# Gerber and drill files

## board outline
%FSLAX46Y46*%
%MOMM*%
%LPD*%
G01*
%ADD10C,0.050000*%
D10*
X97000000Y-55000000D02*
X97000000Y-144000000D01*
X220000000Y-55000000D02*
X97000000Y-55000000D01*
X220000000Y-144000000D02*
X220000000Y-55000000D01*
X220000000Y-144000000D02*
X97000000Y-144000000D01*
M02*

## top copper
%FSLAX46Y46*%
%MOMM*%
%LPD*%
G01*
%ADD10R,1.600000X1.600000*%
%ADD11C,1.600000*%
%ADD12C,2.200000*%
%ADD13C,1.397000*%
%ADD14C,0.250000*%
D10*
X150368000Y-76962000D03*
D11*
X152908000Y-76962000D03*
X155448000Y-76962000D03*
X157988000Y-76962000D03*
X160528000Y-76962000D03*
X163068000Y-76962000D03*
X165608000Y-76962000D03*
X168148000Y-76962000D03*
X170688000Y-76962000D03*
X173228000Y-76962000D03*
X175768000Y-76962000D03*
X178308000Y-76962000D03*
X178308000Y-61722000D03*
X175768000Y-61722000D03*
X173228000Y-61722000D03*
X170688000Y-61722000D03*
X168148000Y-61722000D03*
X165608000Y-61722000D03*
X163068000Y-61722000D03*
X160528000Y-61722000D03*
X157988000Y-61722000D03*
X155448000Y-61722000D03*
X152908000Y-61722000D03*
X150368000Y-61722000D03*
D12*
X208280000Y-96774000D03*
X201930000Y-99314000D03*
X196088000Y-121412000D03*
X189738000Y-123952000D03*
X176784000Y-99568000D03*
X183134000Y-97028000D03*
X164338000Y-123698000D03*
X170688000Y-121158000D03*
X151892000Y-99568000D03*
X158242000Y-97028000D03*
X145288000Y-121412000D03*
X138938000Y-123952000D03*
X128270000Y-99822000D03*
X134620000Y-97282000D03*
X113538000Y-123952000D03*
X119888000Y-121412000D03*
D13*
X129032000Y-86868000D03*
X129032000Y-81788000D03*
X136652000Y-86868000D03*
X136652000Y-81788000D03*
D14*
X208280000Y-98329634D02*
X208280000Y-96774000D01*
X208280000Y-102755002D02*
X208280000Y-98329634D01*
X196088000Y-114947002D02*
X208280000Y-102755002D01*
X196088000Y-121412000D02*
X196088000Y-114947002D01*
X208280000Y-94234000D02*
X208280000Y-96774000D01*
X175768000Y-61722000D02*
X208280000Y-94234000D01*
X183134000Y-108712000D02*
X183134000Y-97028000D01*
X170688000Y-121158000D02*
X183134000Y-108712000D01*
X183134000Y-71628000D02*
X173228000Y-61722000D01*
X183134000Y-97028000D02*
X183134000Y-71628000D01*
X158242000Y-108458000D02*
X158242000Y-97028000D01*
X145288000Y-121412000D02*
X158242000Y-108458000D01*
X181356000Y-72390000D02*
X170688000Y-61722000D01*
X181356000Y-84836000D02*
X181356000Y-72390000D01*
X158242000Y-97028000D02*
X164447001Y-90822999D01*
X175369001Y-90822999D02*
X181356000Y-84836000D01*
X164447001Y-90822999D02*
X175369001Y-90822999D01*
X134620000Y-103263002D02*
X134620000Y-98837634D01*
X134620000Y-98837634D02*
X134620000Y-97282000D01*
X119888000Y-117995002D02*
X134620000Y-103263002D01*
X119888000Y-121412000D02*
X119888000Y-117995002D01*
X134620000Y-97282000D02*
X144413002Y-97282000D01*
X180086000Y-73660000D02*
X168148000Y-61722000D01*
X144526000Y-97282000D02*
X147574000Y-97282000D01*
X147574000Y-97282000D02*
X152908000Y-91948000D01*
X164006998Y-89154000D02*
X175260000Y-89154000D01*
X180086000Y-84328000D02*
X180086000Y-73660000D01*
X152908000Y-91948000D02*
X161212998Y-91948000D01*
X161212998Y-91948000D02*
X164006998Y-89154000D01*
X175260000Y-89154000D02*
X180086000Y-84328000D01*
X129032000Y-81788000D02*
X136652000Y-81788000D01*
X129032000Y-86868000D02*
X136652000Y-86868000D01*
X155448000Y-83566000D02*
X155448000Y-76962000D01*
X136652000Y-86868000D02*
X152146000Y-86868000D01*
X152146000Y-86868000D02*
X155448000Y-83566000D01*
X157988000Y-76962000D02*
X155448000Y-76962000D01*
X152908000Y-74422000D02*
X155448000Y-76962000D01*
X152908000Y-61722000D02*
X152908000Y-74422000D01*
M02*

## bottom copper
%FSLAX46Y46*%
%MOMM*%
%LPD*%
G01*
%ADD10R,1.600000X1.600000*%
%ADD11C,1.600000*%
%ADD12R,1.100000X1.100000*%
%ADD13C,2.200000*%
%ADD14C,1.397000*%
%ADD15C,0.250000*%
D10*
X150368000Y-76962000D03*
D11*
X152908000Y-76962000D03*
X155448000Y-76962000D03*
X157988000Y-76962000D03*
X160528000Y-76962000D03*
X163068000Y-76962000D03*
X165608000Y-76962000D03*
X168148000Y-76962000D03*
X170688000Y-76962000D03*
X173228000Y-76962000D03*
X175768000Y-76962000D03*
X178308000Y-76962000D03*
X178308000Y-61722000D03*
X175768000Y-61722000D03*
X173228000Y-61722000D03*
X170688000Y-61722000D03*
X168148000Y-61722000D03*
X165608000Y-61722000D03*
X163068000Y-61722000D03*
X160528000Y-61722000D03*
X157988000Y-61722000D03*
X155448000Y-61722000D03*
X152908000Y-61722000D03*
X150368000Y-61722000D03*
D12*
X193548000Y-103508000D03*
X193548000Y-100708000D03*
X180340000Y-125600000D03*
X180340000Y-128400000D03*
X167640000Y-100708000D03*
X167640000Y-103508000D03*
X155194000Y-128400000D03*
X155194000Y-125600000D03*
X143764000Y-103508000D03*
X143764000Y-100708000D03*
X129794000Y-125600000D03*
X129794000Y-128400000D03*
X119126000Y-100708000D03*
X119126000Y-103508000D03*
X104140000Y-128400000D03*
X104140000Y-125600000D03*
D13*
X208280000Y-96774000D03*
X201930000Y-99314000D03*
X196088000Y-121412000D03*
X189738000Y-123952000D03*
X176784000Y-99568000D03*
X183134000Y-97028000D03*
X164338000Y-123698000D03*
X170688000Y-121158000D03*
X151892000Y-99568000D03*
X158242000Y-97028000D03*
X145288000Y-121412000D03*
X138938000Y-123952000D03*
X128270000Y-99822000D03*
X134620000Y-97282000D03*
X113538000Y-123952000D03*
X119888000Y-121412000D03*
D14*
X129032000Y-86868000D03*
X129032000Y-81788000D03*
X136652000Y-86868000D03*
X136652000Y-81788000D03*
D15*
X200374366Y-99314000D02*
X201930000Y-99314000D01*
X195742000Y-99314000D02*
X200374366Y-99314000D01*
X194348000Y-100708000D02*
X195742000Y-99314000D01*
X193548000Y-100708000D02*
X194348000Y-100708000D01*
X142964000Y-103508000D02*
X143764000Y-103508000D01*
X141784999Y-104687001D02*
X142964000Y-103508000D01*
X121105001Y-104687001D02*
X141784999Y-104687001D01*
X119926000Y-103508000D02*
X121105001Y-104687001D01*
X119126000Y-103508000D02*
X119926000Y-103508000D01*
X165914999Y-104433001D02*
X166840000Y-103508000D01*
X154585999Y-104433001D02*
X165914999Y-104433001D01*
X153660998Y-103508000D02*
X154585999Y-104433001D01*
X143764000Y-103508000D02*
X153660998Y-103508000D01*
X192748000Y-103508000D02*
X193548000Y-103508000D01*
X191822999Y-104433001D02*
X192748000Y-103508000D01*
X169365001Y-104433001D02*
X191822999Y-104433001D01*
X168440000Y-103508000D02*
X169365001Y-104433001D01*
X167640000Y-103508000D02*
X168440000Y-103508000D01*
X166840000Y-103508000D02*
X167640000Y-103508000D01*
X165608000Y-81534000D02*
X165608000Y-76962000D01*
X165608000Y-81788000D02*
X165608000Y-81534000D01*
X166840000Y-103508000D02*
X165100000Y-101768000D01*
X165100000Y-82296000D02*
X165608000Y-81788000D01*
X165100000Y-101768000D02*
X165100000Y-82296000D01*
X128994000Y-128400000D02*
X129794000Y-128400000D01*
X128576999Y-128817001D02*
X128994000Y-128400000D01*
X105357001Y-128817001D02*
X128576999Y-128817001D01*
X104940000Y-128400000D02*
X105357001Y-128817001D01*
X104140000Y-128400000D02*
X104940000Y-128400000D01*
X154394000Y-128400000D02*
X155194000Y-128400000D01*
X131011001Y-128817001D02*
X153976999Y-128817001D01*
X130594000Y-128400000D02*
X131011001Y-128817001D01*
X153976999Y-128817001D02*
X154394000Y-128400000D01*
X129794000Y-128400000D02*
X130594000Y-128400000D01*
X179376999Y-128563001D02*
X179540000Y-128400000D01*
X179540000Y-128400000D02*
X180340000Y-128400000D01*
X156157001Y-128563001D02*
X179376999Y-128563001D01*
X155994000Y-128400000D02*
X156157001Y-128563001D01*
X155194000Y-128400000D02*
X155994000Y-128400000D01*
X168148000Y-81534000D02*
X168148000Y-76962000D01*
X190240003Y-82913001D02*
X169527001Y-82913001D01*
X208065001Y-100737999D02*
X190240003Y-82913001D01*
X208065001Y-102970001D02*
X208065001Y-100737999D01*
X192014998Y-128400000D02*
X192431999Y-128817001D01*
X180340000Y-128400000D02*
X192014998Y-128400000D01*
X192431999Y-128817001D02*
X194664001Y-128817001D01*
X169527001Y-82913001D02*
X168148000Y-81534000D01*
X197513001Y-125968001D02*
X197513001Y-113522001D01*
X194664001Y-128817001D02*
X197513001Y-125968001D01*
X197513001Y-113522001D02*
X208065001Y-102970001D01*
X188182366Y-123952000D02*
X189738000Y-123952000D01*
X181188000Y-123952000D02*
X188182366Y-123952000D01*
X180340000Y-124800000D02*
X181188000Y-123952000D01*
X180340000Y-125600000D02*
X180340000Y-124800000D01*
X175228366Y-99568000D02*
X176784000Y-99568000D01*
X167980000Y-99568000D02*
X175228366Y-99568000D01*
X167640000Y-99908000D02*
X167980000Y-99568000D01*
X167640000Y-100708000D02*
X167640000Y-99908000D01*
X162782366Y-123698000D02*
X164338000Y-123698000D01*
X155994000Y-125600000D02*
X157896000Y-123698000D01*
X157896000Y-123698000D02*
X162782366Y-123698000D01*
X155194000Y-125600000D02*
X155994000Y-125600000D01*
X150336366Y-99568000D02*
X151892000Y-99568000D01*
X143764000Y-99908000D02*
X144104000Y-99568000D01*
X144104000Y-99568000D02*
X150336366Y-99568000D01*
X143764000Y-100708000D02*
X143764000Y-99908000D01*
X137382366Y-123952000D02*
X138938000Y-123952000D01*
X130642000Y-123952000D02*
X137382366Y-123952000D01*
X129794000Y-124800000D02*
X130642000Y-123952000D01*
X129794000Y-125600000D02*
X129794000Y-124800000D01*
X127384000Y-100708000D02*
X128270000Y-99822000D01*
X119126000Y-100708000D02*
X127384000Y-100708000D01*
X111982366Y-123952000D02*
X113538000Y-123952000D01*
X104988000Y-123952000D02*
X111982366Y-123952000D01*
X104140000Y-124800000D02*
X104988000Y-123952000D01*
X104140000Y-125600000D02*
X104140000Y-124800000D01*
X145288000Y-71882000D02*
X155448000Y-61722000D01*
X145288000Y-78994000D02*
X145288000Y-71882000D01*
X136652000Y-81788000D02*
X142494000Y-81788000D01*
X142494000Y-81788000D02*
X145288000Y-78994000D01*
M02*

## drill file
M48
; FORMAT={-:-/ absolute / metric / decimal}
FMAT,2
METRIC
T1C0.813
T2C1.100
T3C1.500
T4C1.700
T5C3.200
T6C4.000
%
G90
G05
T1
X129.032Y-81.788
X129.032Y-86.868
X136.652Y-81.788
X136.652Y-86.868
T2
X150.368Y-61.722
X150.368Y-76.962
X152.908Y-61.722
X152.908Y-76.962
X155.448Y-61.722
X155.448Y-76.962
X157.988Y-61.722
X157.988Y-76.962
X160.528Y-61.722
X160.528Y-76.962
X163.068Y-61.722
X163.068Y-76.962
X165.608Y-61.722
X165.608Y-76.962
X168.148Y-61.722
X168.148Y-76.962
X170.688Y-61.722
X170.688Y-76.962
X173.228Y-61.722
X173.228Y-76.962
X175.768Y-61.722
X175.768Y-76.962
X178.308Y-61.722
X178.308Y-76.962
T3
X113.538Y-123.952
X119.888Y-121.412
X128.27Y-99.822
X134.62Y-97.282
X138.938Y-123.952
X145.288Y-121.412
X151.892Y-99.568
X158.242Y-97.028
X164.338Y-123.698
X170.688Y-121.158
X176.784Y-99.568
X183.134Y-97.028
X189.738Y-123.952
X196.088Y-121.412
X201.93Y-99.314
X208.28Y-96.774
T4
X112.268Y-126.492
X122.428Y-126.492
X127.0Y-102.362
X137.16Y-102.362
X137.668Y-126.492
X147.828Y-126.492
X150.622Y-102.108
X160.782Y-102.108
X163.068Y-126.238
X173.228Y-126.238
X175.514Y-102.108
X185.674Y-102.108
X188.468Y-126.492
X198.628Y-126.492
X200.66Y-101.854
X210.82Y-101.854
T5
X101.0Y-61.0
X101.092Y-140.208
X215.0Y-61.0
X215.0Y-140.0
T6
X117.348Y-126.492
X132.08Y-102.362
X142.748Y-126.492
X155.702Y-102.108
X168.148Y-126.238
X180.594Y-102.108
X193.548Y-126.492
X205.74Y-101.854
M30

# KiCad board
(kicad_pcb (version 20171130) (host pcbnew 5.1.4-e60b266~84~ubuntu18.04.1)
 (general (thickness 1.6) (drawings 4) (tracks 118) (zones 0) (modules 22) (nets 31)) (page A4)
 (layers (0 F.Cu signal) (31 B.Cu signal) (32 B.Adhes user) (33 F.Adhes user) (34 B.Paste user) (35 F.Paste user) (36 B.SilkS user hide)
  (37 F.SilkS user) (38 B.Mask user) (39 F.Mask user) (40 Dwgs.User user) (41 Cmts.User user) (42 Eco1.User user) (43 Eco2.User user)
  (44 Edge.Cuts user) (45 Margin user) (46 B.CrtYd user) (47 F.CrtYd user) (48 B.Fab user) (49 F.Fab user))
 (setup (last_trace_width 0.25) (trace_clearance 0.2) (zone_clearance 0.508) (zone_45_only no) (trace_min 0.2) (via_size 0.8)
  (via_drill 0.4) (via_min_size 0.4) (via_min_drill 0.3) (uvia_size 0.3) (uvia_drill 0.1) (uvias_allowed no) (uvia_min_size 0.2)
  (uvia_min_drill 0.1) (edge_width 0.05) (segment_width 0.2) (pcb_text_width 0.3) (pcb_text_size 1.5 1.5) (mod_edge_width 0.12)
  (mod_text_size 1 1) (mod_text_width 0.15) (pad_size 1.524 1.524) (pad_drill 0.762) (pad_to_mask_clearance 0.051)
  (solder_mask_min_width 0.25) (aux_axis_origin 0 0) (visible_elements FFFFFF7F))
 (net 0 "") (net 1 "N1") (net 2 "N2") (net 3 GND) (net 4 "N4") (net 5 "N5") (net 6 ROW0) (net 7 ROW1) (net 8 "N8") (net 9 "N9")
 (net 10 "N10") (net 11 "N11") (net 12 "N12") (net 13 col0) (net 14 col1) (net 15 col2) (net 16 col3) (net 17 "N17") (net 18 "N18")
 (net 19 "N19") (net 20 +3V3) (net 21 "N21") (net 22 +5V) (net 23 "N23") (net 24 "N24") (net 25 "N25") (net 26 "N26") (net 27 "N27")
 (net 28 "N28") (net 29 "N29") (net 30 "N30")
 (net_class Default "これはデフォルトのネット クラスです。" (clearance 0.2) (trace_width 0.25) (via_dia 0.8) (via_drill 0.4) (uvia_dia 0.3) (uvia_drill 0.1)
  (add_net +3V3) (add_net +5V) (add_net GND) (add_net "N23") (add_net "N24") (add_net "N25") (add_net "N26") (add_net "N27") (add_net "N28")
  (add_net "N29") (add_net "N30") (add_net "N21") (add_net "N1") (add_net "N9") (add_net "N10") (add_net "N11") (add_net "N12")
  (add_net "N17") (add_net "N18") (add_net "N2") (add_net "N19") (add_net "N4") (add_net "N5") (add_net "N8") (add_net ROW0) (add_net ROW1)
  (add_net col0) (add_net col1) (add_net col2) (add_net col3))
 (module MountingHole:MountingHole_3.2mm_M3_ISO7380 (layer F.Cu) (at 101.092 140.208)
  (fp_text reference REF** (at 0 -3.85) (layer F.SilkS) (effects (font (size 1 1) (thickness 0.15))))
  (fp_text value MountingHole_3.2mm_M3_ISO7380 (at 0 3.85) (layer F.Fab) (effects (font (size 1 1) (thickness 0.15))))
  (pad 1 np_thru_hole circle (at 0 0) (size 3.2 3.2) (drill 3.2) (layers *.Cu *.Mask)))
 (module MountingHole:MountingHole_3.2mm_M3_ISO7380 (layer F.Cu) (at 101 61)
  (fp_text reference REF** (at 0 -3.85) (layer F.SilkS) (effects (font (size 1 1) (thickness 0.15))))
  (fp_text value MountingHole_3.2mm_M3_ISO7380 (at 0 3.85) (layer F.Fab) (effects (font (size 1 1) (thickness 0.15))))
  (pad 1 np_thru_hole circle (at 0 0) (size 3.2 3.2) (drill 3.2) (layers *.Cu *.Mask)))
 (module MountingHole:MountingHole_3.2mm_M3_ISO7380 (layer F.Cu) (at 215 61)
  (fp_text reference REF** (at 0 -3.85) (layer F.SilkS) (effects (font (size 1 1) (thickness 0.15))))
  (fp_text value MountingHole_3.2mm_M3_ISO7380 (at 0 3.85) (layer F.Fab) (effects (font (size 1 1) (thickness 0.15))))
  (pad 1 np_thru_hole circle (at 0 0) (size 3.2 3.2) (drill 3.2) (layers *.Cu *.Mask)))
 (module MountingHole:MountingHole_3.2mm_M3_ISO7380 (layer F.Cu) (at 215 140)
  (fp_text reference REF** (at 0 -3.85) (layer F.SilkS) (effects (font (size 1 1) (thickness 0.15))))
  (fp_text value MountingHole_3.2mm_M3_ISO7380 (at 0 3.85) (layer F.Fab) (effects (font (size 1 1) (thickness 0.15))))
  (pad 1 np_thru_hole circle (at 0 0) (size 3.2 3.2) (drill 3.2) (layers *.Cu *.Mask)))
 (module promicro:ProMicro (layer F.Cu) (at 164.338 69.342)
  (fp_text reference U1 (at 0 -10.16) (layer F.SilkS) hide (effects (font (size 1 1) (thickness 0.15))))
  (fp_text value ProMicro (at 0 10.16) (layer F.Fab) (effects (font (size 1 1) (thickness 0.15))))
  (pad 1 thru_hole rect (at -13.97 7.62) (size 1.6 1.6) (drill 1.1) (layers *.Cu *.Mask F.SilkS) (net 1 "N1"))
  (pad 2 thru_hole circle (at -11.43 7.62) (size 1.6 1.6) (drill 1.1) (layers *.Cu *.Mask F.SilkS) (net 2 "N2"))
  (pad 3 thru_hole circle (at -8.89 7.62) (size 1.6 1.6) (drill 1.1) (layers *.Cu *.Mask F.SilkS) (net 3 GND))
  (pad 4 thru_hole circle (at -6.35 7.62) (size 1.6 1.6) (drill 1.1) (layers *.Cu *.Mask F.SilkS) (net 3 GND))
  (pad 5 thru_hole circle (at -3.81 7.62) (size 1.6 1.6) (drill 1.1) (layers *.Cu *.Mask F.SilkS) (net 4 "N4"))
  (pad 6 thru_hole circle (at -1.27 7.62) (size 1.6 1.6) (drill 1.1) (layers *.Cu *.Mask F.SilkS) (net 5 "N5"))
  (pad 7 thru_hole circle (at 1.27 7.62) (size 1.6 1.6) (drill 1.1) (layers *.Cu *.Mask F.SilkS) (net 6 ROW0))
  (pad 8 thru_hole circle (at 3.81 7.62) (size 1.6 1.6) (drill 1.1) (layers *.Cu *.Mask F.SilkS) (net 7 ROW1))
  (pad 9 thru_hole circle (at 6.35 7.62) (size 1.6 1.6) (drill 1.1) (layers *.Cu *.Mask F.SilkS) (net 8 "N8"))
  (pad 10 thru_hole circle (at 8.89 7.62) (size 1.6 1.6) (drill 1.1) (layers *.Cu *.Mask F.SilkS) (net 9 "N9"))
  (pad 11 thru_hole circle (at 11.43 7.62) (size 1.6 1.6) (drill 1.1) (layers *.Cu *.Mask F.SilkS) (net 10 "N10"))
  (pad 12 thru_hole circle (at 13.97 7.62) (size 1.6 1.6) (drill 1.1) (layers *.Cu *.Mask F.SilkS) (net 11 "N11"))
  (pad 13 thru_hole circle (at 13.97 -7.62) (size 1.6 1.6) (drill 1.1) (layers *.Cu *.Mask F.SilkS) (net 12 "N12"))
  (pad 14 thru_hole circle (at 11.43 -7.62) (size 1.6 1.6) (drill 1.1) (layers *.Cu *.Mask F.SilkS) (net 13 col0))
  (pad 15 thru_hole circle (at 8.89 -7.62) (size 1.6 1.6) (drill 1.1) (layers *.Cu *.Mask F.SilkS) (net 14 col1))
  (pad 16 thru_hole circle (at 6.35 -7.62) (size 1.6 1.6) (drill 1.1) (layers *.Cu *.Mask F.SilkS) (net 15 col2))
  (pad 17 thru_hole circle (at 3.81 -7.62) (size 1.6 1.6) (drill 1.1) (layers *.Cu *.Mask F.SilkS) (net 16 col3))
  (pad 18 thru_hole circle (at 1.27 -7.62) (size 1.6 1.6) (drill 1.1) (layers *.Cu *.Mask F.SilkS) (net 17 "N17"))
  (pad 19 thru_hole circle (at -1.27 -7.62) (size 1.6 1.6) (drill 1.1) (layers *.Cu *.Mask F.SilkS) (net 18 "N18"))
  (pad 20 thru_hole circle (at -3.81 -7.62) (size 1.6 1.6) (drill 1.1) (layers *.Cu *.Mask F.SilkS) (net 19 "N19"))
  (pad 21 thru_hole circle (at -6.35 -7.62) (size 1.6 1.6) (drill 1.1) (layers *.Cu *.Mask F.SilkS) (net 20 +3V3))
  (pad 22 thru_hole circle (at -8.89 -7.62) (size 1.6 1.6) (drill 1.1) (layers *.Cu *.Mask F.SilkS) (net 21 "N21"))
  (pad 23 thru_hole circle (at -11.43 -7.62) (size 1.6 1.6) (drill 1.1) (layers *.Cu *.Mask F.SilkS) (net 3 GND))
  (pad 24 thru_hole circle (at -13.97 -7.62) (size 1.6 1.6) (drill 1.1) (layers *.Cu *.Mask F.SilkS) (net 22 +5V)))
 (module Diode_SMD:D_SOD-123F (layer B.Cu) (at 193.548 102.108 90)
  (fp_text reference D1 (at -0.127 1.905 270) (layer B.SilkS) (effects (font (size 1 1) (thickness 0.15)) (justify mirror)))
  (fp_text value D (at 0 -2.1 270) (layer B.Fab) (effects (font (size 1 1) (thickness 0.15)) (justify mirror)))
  (pad 1 smd rect (at -1.4 0 90) (size 1.1 1.1) (layers B.Cu B.Paste B.Mask) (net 6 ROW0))
  (pad 2 smd rect (at 1.4 0 90) (size 1.1 1.1) (layers B.Cu B.Paste B.Mask) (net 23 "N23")))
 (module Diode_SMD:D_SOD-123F (layer B.Cu) (at 180.34 127 90)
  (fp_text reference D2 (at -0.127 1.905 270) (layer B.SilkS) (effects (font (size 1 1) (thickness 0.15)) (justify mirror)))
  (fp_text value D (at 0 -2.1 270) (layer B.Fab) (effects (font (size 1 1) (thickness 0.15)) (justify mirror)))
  (pad 2 smd rect (at 1.4 0 90) (size 1.1 1.1) (layers B.Cu B.Paste B.Mask) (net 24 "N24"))
  (pad 1 smd rect (at -1.4 0 90) (size 1.1 1.1) (layers B.Cu B.Paste B.Mask) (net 7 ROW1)))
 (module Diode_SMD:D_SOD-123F (layer B.Cu) (at 167.64 102.108 90)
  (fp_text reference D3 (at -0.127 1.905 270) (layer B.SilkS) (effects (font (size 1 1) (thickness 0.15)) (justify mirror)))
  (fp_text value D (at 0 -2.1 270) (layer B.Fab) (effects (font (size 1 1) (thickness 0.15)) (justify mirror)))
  (pad 2 smd rect (at 1.4 0 90) (size 1.1 1.1) (layers B.Cu B.Paste B.Mask) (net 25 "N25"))
  (pad 1 smd rect (at -1.4 0 90) (size 1.1 1.1) (layers B.Cu B.Paste B.Mask) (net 6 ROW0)))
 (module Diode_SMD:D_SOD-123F (layer B.Cu) (at 155.194 127 90)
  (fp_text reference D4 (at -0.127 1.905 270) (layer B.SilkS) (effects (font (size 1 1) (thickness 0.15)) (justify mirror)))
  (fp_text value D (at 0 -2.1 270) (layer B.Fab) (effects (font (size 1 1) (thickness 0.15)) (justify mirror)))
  (pad 1 smd rect (at -1.4 0 90) (size 1.1 1.1) (layers B.Cu B.Paste B.Mask) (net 7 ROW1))
  (pad 2 smd rect (at 1.4 0 90) (size 1.1 1.1) (layers B.Cu B.Paste B.Mask) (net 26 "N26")))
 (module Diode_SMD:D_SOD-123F (layer B.Cu) (at 143.764 102.108 90)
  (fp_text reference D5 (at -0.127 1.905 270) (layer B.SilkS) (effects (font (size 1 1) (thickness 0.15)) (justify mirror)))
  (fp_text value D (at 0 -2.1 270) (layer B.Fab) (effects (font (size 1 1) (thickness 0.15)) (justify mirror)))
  (pad 1 smd rect (at -1.4 0 90) (size 1.1 1.1) (layers B.Cu B.Paste B.Mask) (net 6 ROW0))
  (pad 2 smd rect (at 1.4 0 90) (size 1.1 1.1) (layers B.Cu B.Paste B.Mask) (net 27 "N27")))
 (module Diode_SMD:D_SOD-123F (layer B.Cu) (at 129.794 127 90)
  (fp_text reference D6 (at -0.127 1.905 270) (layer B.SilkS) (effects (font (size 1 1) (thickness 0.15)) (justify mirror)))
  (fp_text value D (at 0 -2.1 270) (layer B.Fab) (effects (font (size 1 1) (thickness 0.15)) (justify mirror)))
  (pad 2 smd rect (at 1.4 0 90) (size 1.1 1.1) (layers B.Cu B.Paste B.Mask) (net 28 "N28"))
  (pad 1 smd rect (at -1.4 0 90) (size 1.1 1.1) (layers B.Cu B.Paste B.Mask) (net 7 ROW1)))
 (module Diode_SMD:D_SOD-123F (layer B.Cu) (at 119.126 102.108 90)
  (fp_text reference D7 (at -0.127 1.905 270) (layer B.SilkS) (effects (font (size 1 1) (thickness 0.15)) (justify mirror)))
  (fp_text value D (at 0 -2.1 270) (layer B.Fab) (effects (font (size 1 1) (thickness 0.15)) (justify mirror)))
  (pad 2 smd rect (at 1.4 0 90) (size 1.1 1.1) (layers B.Cu B.Paste B.Mask) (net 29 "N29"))
  (pad 1 smd rect (at -1.4 0 90) (size 1.1 1.1) (layers B.Cu B.Paste B.Mask) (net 6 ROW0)))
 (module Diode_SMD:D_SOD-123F (layer B.Cu) (at 104.14 127 90)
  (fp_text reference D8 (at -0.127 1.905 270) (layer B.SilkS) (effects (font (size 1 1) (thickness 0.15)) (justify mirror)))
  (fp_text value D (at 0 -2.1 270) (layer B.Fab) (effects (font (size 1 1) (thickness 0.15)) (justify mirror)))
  (pad 1 smd rect (at -1.4 0 90) (size 1.1 1.1) (layers B.Cu B.Paste B.Mask) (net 7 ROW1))
  (pad 2 smd rect (at 1.4 0 90) (size 1.1 1.1) (layers B.Cu B.Paste B.Mask) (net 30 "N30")))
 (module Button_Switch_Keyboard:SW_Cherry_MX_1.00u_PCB (layer F.Cu) (at 208.28 96.774)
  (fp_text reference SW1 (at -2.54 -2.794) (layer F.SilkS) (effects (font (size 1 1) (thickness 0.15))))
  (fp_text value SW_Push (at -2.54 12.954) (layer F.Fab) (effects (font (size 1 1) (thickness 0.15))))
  (pad 1 thru_hole circle (at 0 0) (size 2.2 2.2) (drill 1.5) (layers *.Cu *.Mask) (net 13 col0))
  (pad 2 thru_hole circle (at -6.35 2.54) (size 2.2 2.2) (drill 1.5) (layers *.Cu *.Mask) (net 23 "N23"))
  (pad "" np_thru_hole circle (at -2.54 5.08) (size 4 4) (drill 4) (layers *.Cu *.Mask))
  (pad "" np_thru_hole circle (at -7.62 5.08) (size 1.7 1.7) (drill 1.7) (layers *.Cu *.Mask))
  (pad "" np_thru_hole circle (at 2.54 5.08) (size 1.7 1.7) (drill 1.7) (layers *.Cu *.Mask)))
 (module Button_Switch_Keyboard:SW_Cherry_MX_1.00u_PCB (layer F.Cu) (at 196.088 121.412)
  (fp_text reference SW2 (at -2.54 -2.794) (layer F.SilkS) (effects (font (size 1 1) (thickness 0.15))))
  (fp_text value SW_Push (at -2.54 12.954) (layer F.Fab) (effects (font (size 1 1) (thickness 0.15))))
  (pad 1 thru_hole circle (at 0 0) (size 2.2 2.2) (drill 1.5) (layers *.Cu *.Mask) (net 13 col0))
  (pad 2 thru_hole circle (at -6.35 2.54) (size 2.2 2.2) (drill 1.5) (layers *.Cu *.Mask) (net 24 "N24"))
  (pad "" np_thru_hole circle (at -2.54 5.08) (size 4 4) (drill 4) (layers *.Cu *.Mask))
  (pad "" np_thru_hole circle (at -7.62 5.08) (size 1.7 1.7) (drill 1.7) (layers *.Cu *.Mask))
  (pad "" np_thru_hole circle (at 2.54 5.08) (size 1.7 1.7) (drill 1.7) (layers *.Cu *.Mask)))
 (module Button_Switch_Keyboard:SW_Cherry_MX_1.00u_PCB (layer F.Cu) (at 183.134 97.028)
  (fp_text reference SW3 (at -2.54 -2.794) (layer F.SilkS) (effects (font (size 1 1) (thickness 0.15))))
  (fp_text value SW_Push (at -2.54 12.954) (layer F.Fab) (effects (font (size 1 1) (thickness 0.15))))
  (pad "" np_thru_hole circle (at 2.54 5.08) (size 1.7 1.7) (drill 1.7) (layers *.Cu *.Mask))
  (pad "" np_thru_hole circle (at -7.62 5.08) (size 1.7 1.7) (drill 1.7) (layers *.Cu *.Mask))
  (pad "" np_thru_hole circle (at -2.54 5.08) (size 4 4) (drill 4) (layers *.Cu *.Mask))
  (pad 2 thru_hole circle (at -6.35 2.54) (size 2.2 2.2) (drill 1.5) (layers *.Cu *.Mask) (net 25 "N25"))
  (pad 1 thru_hole circle (at 0 0) (size 2.2 2.2) (drill 1.5) (layers *.Cu *.Mask) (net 14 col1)))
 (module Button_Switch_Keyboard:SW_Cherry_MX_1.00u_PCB (layer F.Cu) (at 170.688 121.158)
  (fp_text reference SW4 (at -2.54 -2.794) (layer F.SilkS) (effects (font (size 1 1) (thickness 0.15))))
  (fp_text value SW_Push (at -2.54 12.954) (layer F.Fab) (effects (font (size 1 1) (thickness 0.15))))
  (pad "" np_thru_hole circle (at 2.54 5.08) (size 1.7 1.7) (drill 1.7) (layers *.Cu *.Mask))
  (pad "" np_thru_hole circle (at -7.62 5.08) (size 1.7 1.7) (drill 1.7) (layers *.Cu *.Mask))
  (pad "" np_thru_hole circle (at -2.54 5.08) (size 4 4) (drill 4) (layers *.Cu *.Mask))
  (pad 2 thru_hole circle (at -6.35 2.54) (size 2.2 2.2) (drill 1.5) (layers *.Cu *.Mask) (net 26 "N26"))
  (pad 1 thru_hole circle (at 0 0) (size 2.2 2.2) (drill 1.5) (layers *.Cu *.Mask) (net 14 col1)))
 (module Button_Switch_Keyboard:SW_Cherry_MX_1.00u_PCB (layer F.Cu) (at 158.242 97.028)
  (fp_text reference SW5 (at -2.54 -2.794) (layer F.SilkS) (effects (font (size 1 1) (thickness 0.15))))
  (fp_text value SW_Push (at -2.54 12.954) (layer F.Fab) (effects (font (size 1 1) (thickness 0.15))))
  (pad "" np_thru_hole circle (at 2.54 5.08) (size 1.7 1.7) (drill 1.7) (layers *.Cu *.Mask))
  (pad "" np_thru_hole circle (at -7.62 5.08) (size 1.7 1.7) (drill 1.7) (layers *.Cu *.Mask))
  (pad "" np_thru_hole circle (at -2.54 5.08) (size 4 4) (drill 4) (layers *.Cu *.Mask))
  (pad 2 thru_hole circle (at -6.35 2.54) (size 2.2 2.2) (drill 1.5) (layers *.Cu *.Mask) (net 27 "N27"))
  (pad 1 thru_hole circle (at 0 0) (size 2.2 2.2) (drill 1.5) (layers *.Cu *.Mask) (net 15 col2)))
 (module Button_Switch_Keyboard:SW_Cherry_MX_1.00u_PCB (layer F.Cu) (at 145.288 121.412)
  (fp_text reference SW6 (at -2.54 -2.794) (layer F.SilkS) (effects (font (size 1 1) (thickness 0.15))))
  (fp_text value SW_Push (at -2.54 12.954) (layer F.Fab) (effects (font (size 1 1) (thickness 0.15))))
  (pad 1 thru_hole circle (at 0 0) (size 2.2 2.2) (drill 1.5) (layers *.Cu *.Mask) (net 15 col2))
  (pad 2 thru_hole circle (at -6.35 2.54) (size 2.2 2.2) (drill 1.5) (layers *.Cu *.Mask) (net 28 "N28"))
  (pad "" np_thru_hole circle (at -2.54 5.08) (size 4 4) (drill 4) (layers *.Cu *.Mask))
  (pad "" np_thru_hole circle (at -7.62 5.08) (size 1.7 1.7) (drill 1.7) (layers *.Cu *.Mask))
  (pad "" np_thru_hole circle (at 2.54 5.08) (size 1.7 1.7) (drill 1.7) (layers *.Cu *.Mask)))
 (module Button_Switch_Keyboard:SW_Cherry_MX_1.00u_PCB (layer F.Cu) (at 134.62 97.282)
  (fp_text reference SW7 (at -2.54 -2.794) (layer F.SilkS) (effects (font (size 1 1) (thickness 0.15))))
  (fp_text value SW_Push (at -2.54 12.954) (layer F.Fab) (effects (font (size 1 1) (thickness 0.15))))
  (pad "" np_thru_hole circle (at 2.54 5.08) (size 1.7 1.7) (drill 1.7) (layers *.Cu *.Mask))
  (pad "" np_thru_hole circle (at -7.62 5.08) (size 1.7 1.7) (drill 1.7) (layers *.Cu *.Mask))
  (pad "" np_thru_hole circle (at -2.54 5.08) (size 4 4) (drill 4) (layers *.Cu *.Mask))
  (pad 2 thru_hole circle (at -6.35 2.54) (size 2.2 2.2) (drill 1.5) (layers *.Cu *.Mask) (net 29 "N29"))
  (pad 1 thru_hole circle (at 0 0) (size 2.2 2.2) (drill 1.5) (layers *.Cu *.Mask) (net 16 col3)))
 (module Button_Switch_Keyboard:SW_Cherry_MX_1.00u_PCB (layer F.Cu) (at 119.888 121.412)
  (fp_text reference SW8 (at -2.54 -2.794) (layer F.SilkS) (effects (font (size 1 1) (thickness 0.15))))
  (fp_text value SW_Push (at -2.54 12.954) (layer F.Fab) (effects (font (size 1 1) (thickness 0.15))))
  (pad "" np_thru_hole circle (at 2.54 5.08) (size 1.7 1.7) (drill 1.7) (layers *.Cu *.Mask))
  (pad "" np_thru_hole circle (at -7.62 5.08) (size 1.7 1.7) (drill 1.7) (layers *.Cu *.Mask))
  (pad "" np_thru_hole circle (at -2.54 5.08) (size 4 4) (drill 4) (layers *.Cu *.Mask))
  (pad 2 thru_hole circle (at -6.35 2.54) (size 2.2 2.2) (drill 1.5) (layers *.Cu *.Mask) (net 30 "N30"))
  (pad 1 thru_hole circle (at 0 0) (size 2.2 2.2) (drill 1.5) (layers *.Cu *.Mask) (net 16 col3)))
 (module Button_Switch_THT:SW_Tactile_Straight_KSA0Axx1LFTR (layer F.Cu) (at 129.032 81.788)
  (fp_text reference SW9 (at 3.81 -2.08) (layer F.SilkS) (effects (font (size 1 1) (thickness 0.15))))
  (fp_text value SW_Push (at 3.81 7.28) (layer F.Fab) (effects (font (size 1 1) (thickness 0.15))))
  (pad 2 thru_hole circle (at 0 5.08) (size 1.397 1.397) (drill 0.8128) (layers *.Cu *.Mask) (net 3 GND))
  (pad 1 thru_hole circle (at 0 0) (size 1.397 1.397) (drill 0.8128) (layers *.Cu *.Mask) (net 21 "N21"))
  (pad 2 thru_hole circle (at 7.62 5.08) (size 1.397 1.397) (drill 0.8128) (layers *.Cu *.Mask) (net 3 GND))
  (pad 1 thru_hole circle (at 7.62 0) (size 1.397 1.397) (drill 0.8128) (layers *.Cu *.Mask) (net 21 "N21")))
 (gr_line (start 97 55) (end 97 144) (layer Edge.Cuts) (width 0.05))
 (gr_line (start 220 55) (end 97 55) (layer Edge.Cuts) (width 0.05))
 (gr_line (start 220 144) (end 220 55) (layer Edge.Cuts) (width 0.05))
 (gr_line (start 220 144) (end 97 144) (layer Edge.Cuts) (width 0.05))
 (segment (start 200.374366 99.314) (end 201.93 99.314) (width 0.25) (layer B.Cu) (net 23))
 (segment (start 195.742 99.314) (end 200.374366 99.314) (width 0.25) (layer B.Cu) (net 23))
 (segment (start 194.348 100.708) (end 195.742 99.314) (width 0.25) (layer B.Cu) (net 23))
 (segment (start 193.548 100.708) (end 194.348 100.708) (width 0.25) (layer B.Cu) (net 23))
 (segment (start 142.964 103.508) (end 143.764 103.508) (width 0.25) (layer B.Cu) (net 6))
 (segment (start 141.784999 104.687001) (end 142.964 103.508) (width 0.25) (layer B.Cu) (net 6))
 (segment (start 121.105001 104.687001) (end 141.784999 104.687001) (width 0.25) (layer B.Cu) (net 6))
 (segment (start 119.926 103.508) (end 121.105001 104.687001) (width 0.25) (layer B.Cu) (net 6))
 (segment (start 119.126 103.508) (end 119.926 103.508) (width 0.25) (layer B.Cu) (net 6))
 (segment (start 165.914999 104.433001) (end 166.84 103.508) (width 0.25) (layer B.Cu) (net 6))
 (segment (start 154.585999 104.433001) (end 165.914999 104.433001) (width 0.25) (layer B.Cu) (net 6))
 (segment (start 153.660998 103.508) (end 154.585999 104.433001) (width 0.25) (layer B.Cu) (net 6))
 (segment (start 143.764 103.508) (end 153.660998 103.508) (width 0.25) (layer B.Cu) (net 6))
 (segment (start 192.748 103.508) (end 193.548 103.508) (width 0.25) (layer B.Cu) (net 6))
 (segment (start 191.822999 104.433001) (end 192.748 103.508) (width 0.25) (layer B.Cu) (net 6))
 (segment (start 169.365001 104.433001) (end 191.822999 104.433001) (width 0.25) (layer B.Cu) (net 6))
 (segment (start 168.44 103.508) (end 169.365001 104.433001) (width 0.25) (layer B.Cu) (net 6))
 (segment (start 167.64 103.508) (end 168.44 103.508) (width 0.25) (layer B.Cu) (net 6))
 (segment (start 166.84 103.508) (end 167.64 103.508) (width 0.25) (layer B.Cu) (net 6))
 (segment (start 165.608 81.534) (end 165.608 76.962) (width 0.25) (layer B.Cu) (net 6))
 (segment (start 165.608 81.788) (end 165.608 81.534) (width 0.25) (layer B.Cu) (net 6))
 (segment (start 166.84 103.508) (end 165.1 101.768) (width 0.25) (layer B.Cu) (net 6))
 (segment (start 165.1 82.296) (end 165.608 81.788) (width 0.25) (layer B.Cu) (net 6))
 (segment (start 165.1 101.768) (end 165.1 82.296) (width 0.25) (layer B.Cu) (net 6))
 (segment (start 128.994 128.4) (end 129.794 128.4) (width 0.25) (layer B.Cu) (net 7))
 (segment (start 128.576999 128.817001) (end 128.994 128.4) (width 0.25) (layer B.Cu) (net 7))
 (segment (start 105.357001 128.817001) (end 128.576999 128.817001) (width 0.25) (layer B.Cu) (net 7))
 (segment (start 104.94 128.4) (end 105.357001 128.817001) (width 0.25) (layer B.Cu) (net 7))
 (segment (start 104.14 128.4) (end 104.94 128.4) (width 0.25) (layer B.Cu) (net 7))
 (segment (start 154.394 128.4) (end 155.194 128.4) (width 0.25) (layer B.Cu) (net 7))
 (segment (start 131.011001 128.817001) (end 153.976999 128.817001) (width 0.25) (layer B.Cu) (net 7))
 (segment (start 130.594 128.4) (end 131.011001 128.817001) (width 0.25) (layer B.Cu) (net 7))
 (segment (start 153.976999 128.817001) (end 154.394 128.4) (width 0.25) (layer B.Cu) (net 7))
 (segment (start 129.794 128.4) (end 130.594 128.4) (width 0.25) (layer B.Cu) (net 7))
 (segment (start 179.376999 128.563001) (end 179.54 128.4) (width 0.25) (layer B.Cu) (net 7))
 (segment (start 179.54 128.4) (end 180.34 128.4) (width 0.25) (layer B.Cu) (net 7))
 (segment (start 156.157001 128.563001) (end 179.376999 128.563001) (width 0.25) (layer B.Cu) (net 7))
 (segment (start 155.994 128.4) (end 156.157001 128.563001) (width 0.25) (layer B.Cu) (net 7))
 (segment (start 155.194 128.4) (end 155.994 128.4) (width 0.25) (layer B.Cu) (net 7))
 (segment (start 168.148 81.534) (end 168.148 76.962) (width 0.25) (layer B.Cu) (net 7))
 (segment (start 190.240003 82.913001) (end 169.527001 82.913001) (width 0.25) (layer B.Cu) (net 7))
 (segment (start 208.065001 100.737999) (end 190.240003 82.913001) (width 0.25) (layer B.Cu) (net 7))
 (segment (start 208.065001 102.970001) (end 208.065001 100.737999) (width 0.25) (layer B.Cu) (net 7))
 (segment (start 192.014998 128.4) (end 192.431999 128.817001) (width 0.25) (layer B.Cu) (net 7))
 (segment (start 180.34 128.4) (end 192.014998 128.4) (width 0.25) (layer B.Cu) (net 7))
 (segment (start 192.431999 128.817001) (end 194.664001 128.817001) (width 0.25) (layer B.Cu) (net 7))
 (segment (start 169.527001 82.913001) (end 168.148 81.534) (width 0.25) (layer B.Cu) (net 7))
 (segment (start 197.513001 125.968001) (end 197.513001 113.522001) (width 0.25) (layer B.Cu) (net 7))
 (segment (start 194.664001 128.817001) (end 197.513001 125.968001) (width 0.25) (layer B.Cu) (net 7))
 (segment (start 197.513001 113.522001) (end 208.065001 102.970001) (width 0.25) (layer B.Cu) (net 7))
 (segment (start 188.182366 123.952) (end 189.738 123.952) (width 0.25) (layer B.Cu) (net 24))
 (segment (start 181.188 123.952) (end 188.182366 123.952) (width 0.25) (layer B.Cu) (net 24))
 (segment (start 180.34 124.8) (end 181.188 123.952) (width 0.25) (layer B.Cu) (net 24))
 (segment (start 180.34 125.6) (end 180.34 124.8) (width 0.25) (layer B.Cu) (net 24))
 (segment (start 175.228366 99.568) (end 176.784 99.568) (width 0.25) (layer B.Cu) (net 25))
 (segment (start 167.98 99.568) (end 175.228366 99.568) (width 0.25) (layer B.Cu) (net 25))
 (segment (start 167.64 99.908) (end 167.98 99.568) (width 0.25) (layer B.Cu) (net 25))
 (segment (start 167.64 100.708) (end 167.64 99.908) (width 0.25) (layer B.Cu) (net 25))
 (segment (start 162.782366 123.698) (end 164.338 123.698) (width 0.25) (layer B.Cu) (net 26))
 (segment (start 155.994 125.6) (end 157.896 123.698) (width 0.25) (layer B.Cu) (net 26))
 (segment (start 157.896 123.698) (end 162.782366 123.698) (width 0.25) (layer B.Cu) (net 26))
 (segment (start 155.194 125.6) (end 155.994 125.6) (width 0.25) (layer B.Cu) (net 26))
 (segment (start 150.336366 99.568) (end 151.892 99.568) (width 0.25) (layer B.Cu) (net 27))
 (segment (start 143.764 99.908) (end 144.104 99.568) (width 0.25) (layer B.Cu) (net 27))
 (segment (start 144.104 99.568) (end 150.336366 99.568) (width 0.25) (layer B.Cu) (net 27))
 (segment (start 143.764 100.708) (end 143.764 99.908) (width 0.25) (layer B.Cu) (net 27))
 (segment (start 137.382366 123.952) (end 138.938 123.952) (width 0.25) (layer B.Cu) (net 28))
 (segment (start 130.642 123.952) (end 137.382366 123.952) (width 0.25) (layer B.Cu) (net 28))
 (segment (start 129.794 124.8) (end 130.642 123.952) (width 0.25) (layer B.Cu) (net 28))
 (segment (start 129.794 125.6) (end 129.794 124.8) (width 0.25) (layer B.Cu) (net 28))
 (segment (start 127.384 100.708) (end 128.27 99.822) (width 0.25) (layer B.Cu) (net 29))
 (segment (start 119.126 100.708) (end 127.384 100.708) (width 0.25) (layer B.Cu) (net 29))
 (segment (start 111.982366 123.952) (end 113.538 123.952) (width 0.25) (layer B.Cu) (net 30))
 (segment (start 104.988 123.952) (end 111.982366 123.952) (width 0.25) (layer B.Cu) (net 30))
 (segment (start 104.14 124.8) (end 104.988 123.952) (width 0.25) (layer B.Cu) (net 30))
 (segment (start 104.14 125.6) (end 104.14 124.8) (width 0.25) (layer B.Cu) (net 30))
 (segment (start 208.28 98.329634) (end 208.28 96.774) (width 0.25) (layer F.Cu) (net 13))
 (segment (start 208.28 102.755002) (end 208.28 98.329634) (width 0.25) (layer F.Cu) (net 13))
 (segment (start 196.088 114.947002) (end 208.28 102.755002) (width 0.25) (layer F.Cu) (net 13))
 (segment (start 196.088 121.412) (end 196.088 114.947002) (width 0.25) (layer F.Cu) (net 13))
 (segment (start 208.28 94.234) (end 208.28 96.774) (width 0.25) (layer F.Cu) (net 13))
 (segment (start 175.768 61.722) (end 208.28 94.234) (width 0.25) (layer F.Cu) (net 13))
 (segment (start 183.134 108.712) (end 183.134 97.028) (width 0.25) (layer F.Cu) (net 14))
 (segment (start 170.688 121.158) (end 183.134 108.712) (width 0.25) (layer F.Cu) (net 14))
 (segment (start 183.134 71.628) (end 173.228 61.722) (width 0.25) (layer F.Cu) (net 14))
 (segment (start 183.134 97.028) (end 183.134 71.628) (width 0.25) (layer F.Cu) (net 14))
 (segment (start 158.242 108.458) (end 158.242 97.028) (width 0.25) (layer F.Cu) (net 15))
 (segment (start 145.288 121.412) (end 158.242 108.458) (width 0.25) (layer F.Cu) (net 15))
 (segment (start 181.356 72.39) (end 170.688 61.722) (width 0.25) (layer F.Cu) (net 15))
 (segment (start 181.356 84.836) (end 181.356 72.39) (width 0.25) (layer F.Cu) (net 15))
 (segment (start 158.242 97.028) (end 164.447001 90.822999) (width 0.25) (layer F.Cu) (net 15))
 (segment (start 175.369001 90.822999) (end 181.356 84.836) (width 0.25) (layer F.Cu) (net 15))
 (segment (start 164.447001 90.822999) (end 175.369001 90.822999) (width 0.25) (layer F.Cu) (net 15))
 (segment (start 134.62 103.263002) (end 134.62 98.837634) (width 0.25) (layer F.Cu) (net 16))
 (segment (start 134.62 98.837634) (end 134.62 97.282) (width 0.25) (layer F.Cu) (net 16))
 (segment (start 119.888 117.995002) (end 134.62 103.263002) (width 0.25) (layer F.Cu) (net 16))
 (segment (start 119.888 121.412) (end 119.888 117.995002) (width 0.25) (layer F.Cu) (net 16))
 (segment (start 134.62 97.282) (end 144.413002 97.282) (width 0.25) (layer F.Cu) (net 16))
 (segment (start 180.086 73.66) (end 168.148 61.722) (width 0.25) (layer F.Cu) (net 16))
 (segment (start 144.526 97.282) (end 147.574 97.282) (width 0.25) (layer F.Cu) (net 16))
 (segment (start 147.574 97.282) (end 152.908 91.948) (width 0.25) (layer F.Cu) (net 16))
 (segment (start 164.006998 89.154) (end 175.26 89.154) (width 0.25) (layer F.Cu) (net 16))
 (segment (start 180.086 84.328) (end 180.086 73.66) (width 0.25) (layer F.Cu) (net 16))
 (segment (start 152.908 91.948) (end 161.212998 91.948) (width 0.25) (layer F.Cu) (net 16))
 (segment (start 161.212998 91.948) (end 164.006998 89.154) (width 0.25) (layer F.Cu) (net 16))
 (segment (start 175.26 89.154) (end 180.086 84.328) (width 0.25) (layer F.Cu) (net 16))
 (segment (start 129.032 81.788) (end 136.652 81.788) (width 0.25) (layer F.Cu) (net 21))
 (segment (start 145.288 71.882) (end 155.448 61.722) (width 0.25) (layer B.Cu) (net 21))
 (segment (start 145.288 78.994) (end 145.288 71.882) (width 0.25) (layer B.Cu) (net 21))
 (segment (start 136.652 81.788) (end 142.494 81.788) (width 0.25) (layer B.Cu) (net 21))
 (segment (start 142.494 81.788) (end 145.288 78.994) (width 0.25) (layer B.Cu) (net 21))
 (segment (start 129.032 86.868) (end 136.652 86.868) (width 0.25) (layer F.Cu) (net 3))
 (segment (start 155.448 83.566) (end 155.448 76.962) (width 0.25) (layer F.Cu) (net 3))
 (segment (start 136.652 86.868) (end 152.146 86.868) (width 0.25) (layer F.Cu) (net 3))
 (segment (start 152.146 86.868) (end 155.448 83.566) (width 0.25) (layer F.Cu) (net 3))
 (segment (start 157.988 76.962) (end 155.448 76.962) (width 0.25) (layer F.Cu) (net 3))
 (segment (start 152.908 74.422) (end 155.448 76.962) (width 0.25) (layer F.Cu) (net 3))
 (segment (start 152.908 61.722) (end 152.908 74.422) (width 0.25) (layer F.Cu) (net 3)))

